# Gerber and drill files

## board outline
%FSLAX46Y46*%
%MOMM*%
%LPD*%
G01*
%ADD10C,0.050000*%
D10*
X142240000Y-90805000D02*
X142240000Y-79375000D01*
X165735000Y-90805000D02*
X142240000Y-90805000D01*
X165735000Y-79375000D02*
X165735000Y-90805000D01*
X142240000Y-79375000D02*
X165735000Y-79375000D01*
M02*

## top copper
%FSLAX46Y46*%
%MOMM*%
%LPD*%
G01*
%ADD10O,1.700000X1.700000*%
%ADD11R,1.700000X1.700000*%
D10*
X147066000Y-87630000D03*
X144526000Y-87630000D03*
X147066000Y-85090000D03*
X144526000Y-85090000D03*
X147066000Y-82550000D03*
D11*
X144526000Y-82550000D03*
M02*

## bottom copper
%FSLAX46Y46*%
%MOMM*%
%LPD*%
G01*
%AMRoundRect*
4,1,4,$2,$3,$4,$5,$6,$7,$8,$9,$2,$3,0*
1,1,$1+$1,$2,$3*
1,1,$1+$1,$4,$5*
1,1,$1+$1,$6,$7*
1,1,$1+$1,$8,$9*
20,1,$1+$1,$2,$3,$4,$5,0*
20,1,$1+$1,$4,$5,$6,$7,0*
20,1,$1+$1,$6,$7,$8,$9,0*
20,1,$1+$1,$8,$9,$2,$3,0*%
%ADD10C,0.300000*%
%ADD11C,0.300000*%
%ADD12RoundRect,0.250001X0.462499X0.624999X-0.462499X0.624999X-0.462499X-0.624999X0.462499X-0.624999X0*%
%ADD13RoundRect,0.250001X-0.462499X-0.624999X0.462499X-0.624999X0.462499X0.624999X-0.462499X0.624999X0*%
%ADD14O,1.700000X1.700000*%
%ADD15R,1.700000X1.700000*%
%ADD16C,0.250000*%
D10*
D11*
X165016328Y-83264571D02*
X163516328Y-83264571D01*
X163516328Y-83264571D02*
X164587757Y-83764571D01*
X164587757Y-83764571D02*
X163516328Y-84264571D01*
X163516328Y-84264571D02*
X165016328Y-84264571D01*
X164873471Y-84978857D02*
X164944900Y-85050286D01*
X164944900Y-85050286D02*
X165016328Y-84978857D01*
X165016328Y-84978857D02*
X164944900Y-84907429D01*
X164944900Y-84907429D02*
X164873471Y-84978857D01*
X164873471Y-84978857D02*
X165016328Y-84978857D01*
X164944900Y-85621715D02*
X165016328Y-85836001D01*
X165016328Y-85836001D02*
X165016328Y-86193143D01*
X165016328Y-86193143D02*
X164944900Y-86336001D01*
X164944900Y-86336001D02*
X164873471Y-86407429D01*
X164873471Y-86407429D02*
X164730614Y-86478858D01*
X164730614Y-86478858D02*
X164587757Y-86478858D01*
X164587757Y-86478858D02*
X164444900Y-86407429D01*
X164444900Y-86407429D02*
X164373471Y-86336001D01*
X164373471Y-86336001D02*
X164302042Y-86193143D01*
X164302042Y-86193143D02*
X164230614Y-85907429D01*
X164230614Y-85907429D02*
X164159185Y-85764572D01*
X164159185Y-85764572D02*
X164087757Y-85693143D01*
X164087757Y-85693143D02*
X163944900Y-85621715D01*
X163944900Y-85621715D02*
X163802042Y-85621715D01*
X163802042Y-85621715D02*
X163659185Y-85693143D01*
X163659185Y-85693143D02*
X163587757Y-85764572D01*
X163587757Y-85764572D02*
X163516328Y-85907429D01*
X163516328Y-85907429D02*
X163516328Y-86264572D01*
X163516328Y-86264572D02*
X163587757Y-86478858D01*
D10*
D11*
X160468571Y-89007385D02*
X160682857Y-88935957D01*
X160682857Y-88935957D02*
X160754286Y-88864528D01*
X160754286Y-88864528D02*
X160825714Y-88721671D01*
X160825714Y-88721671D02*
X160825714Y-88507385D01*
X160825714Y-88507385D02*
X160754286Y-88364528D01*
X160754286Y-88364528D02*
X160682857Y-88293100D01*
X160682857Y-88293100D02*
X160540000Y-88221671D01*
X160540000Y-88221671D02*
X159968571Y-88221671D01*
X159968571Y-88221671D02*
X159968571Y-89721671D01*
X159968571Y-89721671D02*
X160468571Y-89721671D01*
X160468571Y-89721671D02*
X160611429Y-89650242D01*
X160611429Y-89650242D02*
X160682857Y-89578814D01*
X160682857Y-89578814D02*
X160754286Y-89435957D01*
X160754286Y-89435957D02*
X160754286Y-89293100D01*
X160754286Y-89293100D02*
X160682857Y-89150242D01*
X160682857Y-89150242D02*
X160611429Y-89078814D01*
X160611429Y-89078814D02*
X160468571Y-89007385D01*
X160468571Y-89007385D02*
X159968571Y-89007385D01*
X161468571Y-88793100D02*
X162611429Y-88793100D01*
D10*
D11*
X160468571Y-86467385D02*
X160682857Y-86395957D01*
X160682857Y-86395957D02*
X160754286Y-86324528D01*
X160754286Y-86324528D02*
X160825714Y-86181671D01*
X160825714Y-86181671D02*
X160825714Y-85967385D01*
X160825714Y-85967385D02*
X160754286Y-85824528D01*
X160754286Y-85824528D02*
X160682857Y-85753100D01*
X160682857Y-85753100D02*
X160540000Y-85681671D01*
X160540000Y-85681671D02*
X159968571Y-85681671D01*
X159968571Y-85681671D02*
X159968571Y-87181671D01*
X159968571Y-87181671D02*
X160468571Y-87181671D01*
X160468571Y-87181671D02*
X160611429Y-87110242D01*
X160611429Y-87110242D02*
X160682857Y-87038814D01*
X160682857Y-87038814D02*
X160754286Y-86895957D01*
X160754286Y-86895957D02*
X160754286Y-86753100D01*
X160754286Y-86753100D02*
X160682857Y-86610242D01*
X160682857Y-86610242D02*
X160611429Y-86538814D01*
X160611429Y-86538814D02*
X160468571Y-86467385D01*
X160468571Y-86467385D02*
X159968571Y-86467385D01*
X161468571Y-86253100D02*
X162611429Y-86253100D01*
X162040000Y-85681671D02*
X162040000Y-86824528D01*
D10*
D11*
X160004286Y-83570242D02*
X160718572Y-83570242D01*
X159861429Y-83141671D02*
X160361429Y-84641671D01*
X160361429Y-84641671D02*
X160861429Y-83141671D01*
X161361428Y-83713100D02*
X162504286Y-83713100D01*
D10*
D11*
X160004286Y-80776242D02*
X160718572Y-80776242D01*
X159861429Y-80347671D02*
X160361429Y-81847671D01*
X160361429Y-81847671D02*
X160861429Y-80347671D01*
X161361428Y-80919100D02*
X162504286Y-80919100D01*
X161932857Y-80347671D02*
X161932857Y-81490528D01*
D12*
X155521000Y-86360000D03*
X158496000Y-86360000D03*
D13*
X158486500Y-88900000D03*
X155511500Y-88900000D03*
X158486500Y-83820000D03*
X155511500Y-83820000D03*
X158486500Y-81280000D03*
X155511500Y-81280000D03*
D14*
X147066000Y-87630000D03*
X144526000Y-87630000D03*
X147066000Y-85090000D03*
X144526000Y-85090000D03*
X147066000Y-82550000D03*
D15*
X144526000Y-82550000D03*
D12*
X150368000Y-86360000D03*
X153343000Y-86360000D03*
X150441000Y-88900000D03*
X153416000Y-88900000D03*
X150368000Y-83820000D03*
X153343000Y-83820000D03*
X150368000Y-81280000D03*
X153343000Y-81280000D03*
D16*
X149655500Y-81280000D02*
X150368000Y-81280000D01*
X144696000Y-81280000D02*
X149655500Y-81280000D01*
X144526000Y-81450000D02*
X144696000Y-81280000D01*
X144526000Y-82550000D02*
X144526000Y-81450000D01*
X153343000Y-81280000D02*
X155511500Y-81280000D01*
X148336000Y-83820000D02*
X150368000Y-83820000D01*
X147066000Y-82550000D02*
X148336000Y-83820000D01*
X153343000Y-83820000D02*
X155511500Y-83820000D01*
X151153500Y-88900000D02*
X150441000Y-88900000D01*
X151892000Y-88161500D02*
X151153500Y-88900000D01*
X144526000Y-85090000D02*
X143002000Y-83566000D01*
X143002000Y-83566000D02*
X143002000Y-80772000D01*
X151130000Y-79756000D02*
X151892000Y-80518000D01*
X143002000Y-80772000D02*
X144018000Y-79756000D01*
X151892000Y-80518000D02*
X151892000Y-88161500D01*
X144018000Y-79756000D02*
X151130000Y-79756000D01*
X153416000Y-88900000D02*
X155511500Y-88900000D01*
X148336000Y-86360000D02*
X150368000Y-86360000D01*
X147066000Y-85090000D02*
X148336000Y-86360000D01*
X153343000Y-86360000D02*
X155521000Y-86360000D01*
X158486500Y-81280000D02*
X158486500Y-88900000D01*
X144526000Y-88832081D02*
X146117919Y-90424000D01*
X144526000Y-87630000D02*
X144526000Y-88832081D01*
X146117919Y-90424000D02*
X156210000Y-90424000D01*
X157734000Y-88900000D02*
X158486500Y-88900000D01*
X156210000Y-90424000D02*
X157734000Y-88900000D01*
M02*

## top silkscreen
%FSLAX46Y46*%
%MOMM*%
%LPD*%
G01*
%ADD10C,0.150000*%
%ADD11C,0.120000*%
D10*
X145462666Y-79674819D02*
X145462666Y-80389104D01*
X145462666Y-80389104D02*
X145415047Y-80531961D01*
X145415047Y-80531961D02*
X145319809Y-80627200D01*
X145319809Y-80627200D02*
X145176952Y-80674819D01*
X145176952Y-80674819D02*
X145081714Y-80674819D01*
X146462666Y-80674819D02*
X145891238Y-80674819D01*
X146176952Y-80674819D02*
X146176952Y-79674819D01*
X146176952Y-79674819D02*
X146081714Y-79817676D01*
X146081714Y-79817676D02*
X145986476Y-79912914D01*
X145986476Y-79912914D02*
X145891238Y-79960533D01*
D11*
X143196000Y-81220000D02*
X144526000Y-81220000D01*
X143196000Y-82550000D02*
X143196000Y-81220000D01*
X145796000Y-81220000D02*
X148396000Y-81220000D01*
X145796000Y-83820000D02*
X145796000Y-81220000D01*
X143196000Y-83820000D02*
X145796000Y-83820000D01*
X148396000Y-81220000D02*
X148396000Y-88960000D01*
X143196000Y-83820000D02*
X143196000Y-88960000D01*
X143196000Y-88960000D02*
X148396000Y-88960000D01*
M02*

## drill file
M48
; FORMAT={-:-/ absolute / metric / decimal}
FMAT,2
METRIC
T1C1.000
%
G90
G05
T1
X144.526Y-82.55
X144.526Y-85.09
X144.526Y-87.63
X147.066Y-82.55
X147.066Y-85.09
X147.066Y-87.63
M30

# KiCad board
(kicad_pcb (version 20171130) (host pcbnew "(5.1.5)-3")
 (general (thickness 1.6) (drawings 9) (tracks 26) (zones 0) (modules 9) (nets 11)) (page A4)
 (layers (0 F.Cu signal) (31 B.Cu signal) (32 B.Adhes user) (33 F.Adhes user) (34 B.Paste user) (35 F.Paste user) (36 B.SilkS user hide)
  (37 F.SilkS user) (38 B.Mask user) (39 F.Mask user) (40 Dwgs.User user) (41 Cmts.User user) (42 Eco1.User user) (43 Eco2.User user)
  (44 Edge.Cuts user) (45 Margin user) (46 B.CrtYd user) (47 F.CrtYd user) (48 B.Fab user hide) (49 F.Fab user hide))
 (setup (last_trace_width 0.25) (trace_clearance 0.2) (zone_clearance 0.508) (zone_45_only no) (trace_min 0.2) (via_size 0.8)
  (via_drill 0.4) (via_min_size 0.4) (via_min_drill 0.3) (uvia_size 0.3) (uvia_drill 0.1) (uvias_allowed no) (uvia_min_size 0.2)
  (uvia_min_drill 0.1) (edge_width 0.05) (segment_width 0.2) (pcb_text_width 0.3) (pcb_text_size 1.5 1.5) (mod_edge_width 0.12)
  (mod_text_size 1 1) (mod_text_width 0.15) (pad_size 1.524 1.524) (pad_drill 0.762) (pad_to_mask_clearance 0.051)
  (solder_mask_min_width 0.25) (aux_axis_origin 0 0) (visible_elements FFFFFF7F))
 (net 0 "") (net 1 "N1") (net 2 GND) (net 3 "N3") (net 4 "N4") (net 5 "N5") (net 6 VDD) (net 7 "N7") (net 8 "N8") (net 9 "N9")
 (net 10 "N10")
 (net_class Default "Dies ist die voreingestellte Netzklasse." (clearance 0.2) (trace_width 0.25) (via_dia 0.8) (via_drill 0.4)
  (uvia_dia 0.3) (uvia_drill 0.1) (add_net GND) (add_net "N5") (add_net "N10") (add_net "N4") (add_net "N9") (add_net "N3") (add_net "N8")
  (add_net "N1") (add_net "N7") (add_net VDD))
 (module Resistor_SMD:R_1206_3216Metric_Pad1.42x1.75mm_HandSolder (layer B.Cu) (at 157.0085 86.36 180)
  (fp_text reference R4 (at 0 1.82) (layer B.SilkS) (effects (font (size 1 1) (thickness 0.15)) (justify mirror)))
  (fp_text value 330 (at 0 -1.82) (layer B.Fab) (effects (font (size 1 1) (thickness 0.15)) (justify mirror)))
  (pad 2 smd roundrect (at 1.4875 0 180) (size 1.425 1.75) (layers B.Cu B.Paste B.Mask) (roundrect_rratio 0.175439) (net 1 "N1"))
  (pad 1 smd roundrect (at -1.4875 0 180) (size 1.425 1.75) (layers B.Cu B.Paste B.Mask) (roundrect_rratio 0.175439) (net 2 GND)))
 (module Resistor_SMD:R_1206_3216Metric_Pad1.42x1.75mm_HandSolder (layer B.Cu) (at 156.999 88.9)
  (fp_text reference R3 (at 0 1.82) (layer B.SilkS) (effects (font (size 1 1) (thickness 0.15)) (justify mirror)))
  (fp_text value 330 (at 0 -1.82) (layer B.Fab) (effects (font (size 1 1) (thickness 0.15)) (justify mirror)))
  (pad 2 smd roundrect (at 1.4875 0) (size 1.425 1.75) (layers B.Cu B.Paste B.Mask) (roundrect_rratio 0.175439) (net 2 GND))
  (pad 1 smd roundrect (at -1.4875 0) (size 1.425 1.75) (layers B.Cu B.Paste B.Mask) (roundrect_rratio 0.175439) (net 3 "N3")))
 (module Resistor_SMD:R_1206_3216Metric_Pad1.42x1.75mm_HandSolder (layer B.Cu) (at 156.999 83.82)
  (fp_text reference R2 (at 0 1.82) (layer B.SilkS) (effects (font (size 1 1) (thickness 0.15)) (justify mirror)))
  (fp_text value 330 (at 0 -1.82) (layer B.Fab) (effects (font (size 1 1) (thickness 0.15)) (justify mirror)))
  (pad 2 smd roundrect (at 1.4875 0) (size 1.425 1.75) (layers B.Cu B.Paste B.Mask) (roundrect_rratio 0.175439) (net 2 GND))
  (pad 1 smd roundrect (at -1.4875 0) (size 1.425 1.75) (layers B.Cu B.Paste B.Mask) (roundrect_rratio 0.175439) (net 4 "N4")))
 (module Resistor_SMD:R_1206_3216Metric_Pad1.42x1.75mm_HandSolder (layer B.Cu) (at 156.999 81.28)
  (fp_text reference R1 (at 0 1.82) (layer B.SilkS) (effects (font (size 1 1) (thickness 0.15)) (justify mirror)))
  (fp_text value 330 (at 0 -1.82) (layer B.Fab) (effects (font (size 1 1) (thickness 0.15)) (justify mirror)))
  (pad 2 smd roundrect (at 1.4875 0) (size 1.425 1.75) (layers B.Cu B.Paste B.Mask) (roundrect_rratio 0.175439) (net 2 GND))
  (pad 1 smd roundrect (at -1.4875 0) (size 1.425 1.75) (layers B.Cu B.Paste B.Mask) (roundrect_rratio 0.175439) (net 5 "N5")))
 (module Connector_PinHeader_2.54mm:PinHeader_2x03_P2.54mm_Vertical (layer F.Cu) (at 144.526 82.55)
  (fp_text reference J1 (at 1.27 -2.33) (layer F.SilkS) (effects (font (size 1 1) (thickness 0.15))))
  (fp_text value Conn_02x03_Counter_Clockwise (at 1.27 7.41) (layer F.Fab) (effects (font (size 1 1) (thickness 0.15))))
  (fp_line (start -1.33 -1.33) (end 0 -1.33) (layer F.SilkS) (width 0.12))
  (fp_line (start -1.33 0) (end -1.33 -1.33) (layer F.SilkS) (width 0.12))
  (fp_line (start 1.27 -1.33) (end 3.87 -1.33) (layer F.SilkS) (width 0.12))
  (fp_line (start 1.27 1.27) (end 1.27 -1.33) (layer F.SilkS) (width 0.12))
  (fp_line (start -1.33 1.27) (end 1.27 1.27) (layer F.SilkS) (width 0.12))
  (fp_line (start 3.87 -1.33) (end 3.87 6.41) (layer F.SilkS) (width 0.12))
  (fp_line (start -1.33 1.27) (end -1.33 6.41) (layer F.SilkS) (width 0.12))
  (fp_line (start -1.33 6.41) (end 3.87 6.41) (layer F.SilkS) (width 0.12))
  (pad 6 thru_hole oval (at 2.54 5.08) (size 1.7 1.7) (drill 1) (layers *.Cu *.Mask) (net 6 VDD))
  (pad 5 thru_hole oval (at 0 5.08) (size 1.7 1.7) (drill 1) (layers *.Cu *.Mask) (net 2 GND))
  (pad 4 thru_hole oval (at 2.54 2.54) (size 1.7 1.7) (drill 1) (layers *.Cu *.Mask) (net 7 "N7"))
  (pad 3 thru_hole oval (at 0 2.54) (size 1.7 1.7) (drill 1) (layers *.Cu *.Mask) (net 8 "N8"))
  (pad 2 thru_hole oval (at 2.54 0) (size 1.7 1.7) (drill 1) (layers *.Cu *.Mask) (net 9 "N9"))
  (pad 1 thru_hole rect (at 0 0) (size 1.7 1.7) (drill 1) (layers *.Cu *.Mask) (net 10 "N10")))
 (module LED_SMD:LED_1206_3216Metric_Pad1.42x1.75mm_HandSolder (layer B.Cu) (at 151.8555 86.36 180)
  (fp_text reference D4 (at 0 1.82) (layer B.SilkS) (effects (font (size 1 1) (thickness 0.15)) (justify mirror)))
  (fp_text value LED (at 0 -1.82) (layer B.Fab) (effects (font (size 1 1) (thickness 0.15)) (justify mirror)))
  (pad 2 smd roundrect (at 1.4875 0 180) (size 1.425 1.75) (layers B.Cu B.Paste B.Mask) (roundrect_rratio 0.175439) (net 7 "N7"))
  (pad 1 smd roundrect (at -1.4875 0 180) (size 1.425 1.75) (layers B.Cu B.Paste B.Mask) (roundrect_rratio 0.175439) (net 1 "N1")))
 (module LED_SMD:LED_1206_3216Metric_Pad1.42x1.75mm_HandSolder (layer B.Cu) (at 151.9285 88.9 180)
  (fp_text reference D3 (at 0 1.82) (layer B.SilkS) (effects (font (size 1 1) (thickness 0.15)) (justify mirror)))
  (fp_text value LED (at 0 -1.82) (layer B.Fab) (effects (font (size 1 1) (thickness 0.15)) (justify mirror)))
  (pad 2 smd roundrect (at 1.4875 0 180) (size 1.425 1.75) (layers B.Cu B.Paste B.Mask) (roundrect_rratio 0.175439) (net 8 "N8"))
  (pad 1 smd roundrect (at -1.4875 0 180) (size 1.425 1.75) (layers B.Cu B.Paste B.Mask) (roundrect_rratio 0.175439) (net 3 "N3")))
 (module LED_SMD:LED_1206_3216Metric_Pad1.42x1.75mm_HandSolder (layer B.Cu) (at 151.8555 83.82 180)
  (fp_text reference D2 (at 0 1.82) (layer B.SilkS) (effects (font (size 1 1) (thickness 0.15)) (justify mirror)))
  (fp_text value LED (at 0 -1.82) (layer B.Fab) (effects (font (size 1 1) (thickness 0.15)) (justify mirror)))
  (pad 2 smd roundrect (at 1.4875 0 180) (size 1.425 1.75) (layers B.Cu B.Paste B.Mask) (roundrect_rratio 0.175439) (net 9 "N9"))
  (pad 1 smd roundrect (at -1.4875 0 180) (size 1.425 1.75) (layers B.Cu B.Paste B.Mask) (roundrect_rratio 0.175439) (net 4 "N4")))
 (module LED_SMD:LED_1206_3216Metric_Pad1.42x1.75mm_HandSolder (layer B.Cu) (at 151.8555 81.28 180)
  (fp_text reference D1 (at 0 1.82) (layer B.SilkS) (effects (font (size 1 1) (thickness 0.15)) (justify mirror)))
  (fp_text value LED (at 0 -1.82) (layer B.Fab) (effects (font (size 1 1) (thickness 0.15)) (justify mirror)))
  (pad 2 smd roundrect (at 1.4875 0 180) (size 1.425 1.75) (layers B.Cu B.Paste B.Mask) (roundrect_rratio 0.175439) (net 10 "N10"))
  (pad 1 smd roundrect (at -1.4875 0 180) (size 1.425 1.75) (layers B.Cu B.Paste B.Mask) (roundrect_rratio 0.175439) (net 5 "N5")))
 (gr_line (start 142.24 90.805) (end 142.24 79.375) (layer Edge.Cuts) (width 0.05))
 (gr_line (start 165.735 90.805) (end 142.24 90.805) (layer Edge.Cuts) (width 0.05))
 (gr_line (start 165.735 79.375) (end 165.735 90.805) (layer Edge.Cuts) (width 0.05))
 (gr_line (start 142.24 79.375) (end 165.735 79.375) (layer Edge.Cuts) (width 0.05))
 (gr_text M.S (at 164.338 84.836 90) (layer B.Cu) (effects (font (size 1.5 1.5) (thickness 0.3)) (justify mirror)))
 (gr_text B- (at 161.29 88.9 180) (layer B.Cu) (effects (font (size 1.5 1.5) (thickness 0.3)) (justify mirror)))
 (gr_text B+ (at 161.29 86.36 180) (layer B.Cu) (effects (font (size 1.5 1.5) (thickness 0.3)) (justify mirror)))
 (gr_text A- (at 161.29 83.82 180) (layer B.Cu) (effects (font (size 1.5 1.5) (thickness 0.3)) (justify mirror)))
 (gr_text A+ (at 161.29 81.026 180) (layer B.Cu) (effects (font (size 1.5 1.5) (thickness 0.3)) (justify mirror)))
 (segment (start 149.6555 81.28) (end 150.368 81.28) (width 0.25) (layer B.Cu) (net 10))
 (segment (start 144.696 81.28) (end 149.6555 81.28) (width 0.25) (layer B.Cu) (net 10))
 (segment (start 144.526 81.45) (end 144.696 81.28) (width 0.25) (layer B.Cu) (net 10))
 (segment (start 144.526 82.55) (end 144.526 81.45) (width 0.25) (layer B.Cu) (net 10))
 (segment (start 153.343 81.28) (end 155.5115 81.28) (width 0.25) (layer B.Cu) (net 5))
 (segment (start 148.336 83.82) (end 150.368 83.82) (width 0.25) (layer B.Cu) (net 9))
 (segment (start 147.066 82.55) (end 148.336 83.82) (width 0.25) (layer B.Cu) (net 9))
 (segment (start 153.343 83.82) (end 155.5115 83.82) (width 0.25) (layer B.Cu) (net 4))
 (segment (start 151.1535 88.9) (end 150.441 88.9) (width 0.25) (layer B.Cu) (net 8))
 (segment (start 151.892 88.1615) (end 151.1535 88.9) (width 0.25) (layer B.Cu) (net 8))
 (segment (start 144.526 85.09) (end 143.002 83.566) (width 0.25) (layer B.Cu) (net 8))
 (segment (start 143.002 83.566) (end 143.002 80.772) (width 0.25) (layer B.Cu) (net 8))
 (segment (start 151.13 79.756) (end 151.892 80.518) (width 0.25) (layer B.Cu) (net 8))
 (segment (start 143.002 80.772) (end 144.018 79.756) (width 0.25) (layer B.Cu) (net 8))
 (segment (start 151.892 80.518) (end 151.892 88.1615) (width 0.25) (layer B.Cu) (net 8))
 (segment (start 144.018 79.756) (end 151.13 79.756) (width 0.25) (layer B.Cu) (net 8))
 (segment (start 153.416 88.9) (end 155.5115 88.9) (width 0.25) (layer B.Cu) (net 3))
 (segment (start 148.336 86.36) (end 150.368 86.36) (width 0.25) (layer B.Cu) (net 7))
 (segment (start 147.066 85.09) (end 148.336 86.36) (width 0.25) (layer B.Cu) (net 7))
 (segment (start 153.343 86.36) (end 155.521 86.36) (width 0.25) (layer B.Cu) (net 1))
 (segment (start 158.4865 81.28) (end 158.4865 88.9) (width 0.25) (layer B.Cu) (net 2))
 (segment (start 144.526 88.832081) (end 146.117919 90.424) (width 0.25) (layer B.Cu) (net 2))
 (segment (start 144.526 87.63) (end 144.526 88.832081) (width 0.25) (layer B.Cu) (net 2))
 (segment (start 146.117919 90.424) (end 156.21 90.424) (width 0.25) (layer B.Cu) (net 2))
 (segment (start 157.734 88.9) (end 158.4865 88.9) (width 0.25) (layer B.Cu) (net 2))
 (segment (start 156.21 90.424) (end 157.734 88.9) (width 0.25) (layer B.Cu) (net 2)))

